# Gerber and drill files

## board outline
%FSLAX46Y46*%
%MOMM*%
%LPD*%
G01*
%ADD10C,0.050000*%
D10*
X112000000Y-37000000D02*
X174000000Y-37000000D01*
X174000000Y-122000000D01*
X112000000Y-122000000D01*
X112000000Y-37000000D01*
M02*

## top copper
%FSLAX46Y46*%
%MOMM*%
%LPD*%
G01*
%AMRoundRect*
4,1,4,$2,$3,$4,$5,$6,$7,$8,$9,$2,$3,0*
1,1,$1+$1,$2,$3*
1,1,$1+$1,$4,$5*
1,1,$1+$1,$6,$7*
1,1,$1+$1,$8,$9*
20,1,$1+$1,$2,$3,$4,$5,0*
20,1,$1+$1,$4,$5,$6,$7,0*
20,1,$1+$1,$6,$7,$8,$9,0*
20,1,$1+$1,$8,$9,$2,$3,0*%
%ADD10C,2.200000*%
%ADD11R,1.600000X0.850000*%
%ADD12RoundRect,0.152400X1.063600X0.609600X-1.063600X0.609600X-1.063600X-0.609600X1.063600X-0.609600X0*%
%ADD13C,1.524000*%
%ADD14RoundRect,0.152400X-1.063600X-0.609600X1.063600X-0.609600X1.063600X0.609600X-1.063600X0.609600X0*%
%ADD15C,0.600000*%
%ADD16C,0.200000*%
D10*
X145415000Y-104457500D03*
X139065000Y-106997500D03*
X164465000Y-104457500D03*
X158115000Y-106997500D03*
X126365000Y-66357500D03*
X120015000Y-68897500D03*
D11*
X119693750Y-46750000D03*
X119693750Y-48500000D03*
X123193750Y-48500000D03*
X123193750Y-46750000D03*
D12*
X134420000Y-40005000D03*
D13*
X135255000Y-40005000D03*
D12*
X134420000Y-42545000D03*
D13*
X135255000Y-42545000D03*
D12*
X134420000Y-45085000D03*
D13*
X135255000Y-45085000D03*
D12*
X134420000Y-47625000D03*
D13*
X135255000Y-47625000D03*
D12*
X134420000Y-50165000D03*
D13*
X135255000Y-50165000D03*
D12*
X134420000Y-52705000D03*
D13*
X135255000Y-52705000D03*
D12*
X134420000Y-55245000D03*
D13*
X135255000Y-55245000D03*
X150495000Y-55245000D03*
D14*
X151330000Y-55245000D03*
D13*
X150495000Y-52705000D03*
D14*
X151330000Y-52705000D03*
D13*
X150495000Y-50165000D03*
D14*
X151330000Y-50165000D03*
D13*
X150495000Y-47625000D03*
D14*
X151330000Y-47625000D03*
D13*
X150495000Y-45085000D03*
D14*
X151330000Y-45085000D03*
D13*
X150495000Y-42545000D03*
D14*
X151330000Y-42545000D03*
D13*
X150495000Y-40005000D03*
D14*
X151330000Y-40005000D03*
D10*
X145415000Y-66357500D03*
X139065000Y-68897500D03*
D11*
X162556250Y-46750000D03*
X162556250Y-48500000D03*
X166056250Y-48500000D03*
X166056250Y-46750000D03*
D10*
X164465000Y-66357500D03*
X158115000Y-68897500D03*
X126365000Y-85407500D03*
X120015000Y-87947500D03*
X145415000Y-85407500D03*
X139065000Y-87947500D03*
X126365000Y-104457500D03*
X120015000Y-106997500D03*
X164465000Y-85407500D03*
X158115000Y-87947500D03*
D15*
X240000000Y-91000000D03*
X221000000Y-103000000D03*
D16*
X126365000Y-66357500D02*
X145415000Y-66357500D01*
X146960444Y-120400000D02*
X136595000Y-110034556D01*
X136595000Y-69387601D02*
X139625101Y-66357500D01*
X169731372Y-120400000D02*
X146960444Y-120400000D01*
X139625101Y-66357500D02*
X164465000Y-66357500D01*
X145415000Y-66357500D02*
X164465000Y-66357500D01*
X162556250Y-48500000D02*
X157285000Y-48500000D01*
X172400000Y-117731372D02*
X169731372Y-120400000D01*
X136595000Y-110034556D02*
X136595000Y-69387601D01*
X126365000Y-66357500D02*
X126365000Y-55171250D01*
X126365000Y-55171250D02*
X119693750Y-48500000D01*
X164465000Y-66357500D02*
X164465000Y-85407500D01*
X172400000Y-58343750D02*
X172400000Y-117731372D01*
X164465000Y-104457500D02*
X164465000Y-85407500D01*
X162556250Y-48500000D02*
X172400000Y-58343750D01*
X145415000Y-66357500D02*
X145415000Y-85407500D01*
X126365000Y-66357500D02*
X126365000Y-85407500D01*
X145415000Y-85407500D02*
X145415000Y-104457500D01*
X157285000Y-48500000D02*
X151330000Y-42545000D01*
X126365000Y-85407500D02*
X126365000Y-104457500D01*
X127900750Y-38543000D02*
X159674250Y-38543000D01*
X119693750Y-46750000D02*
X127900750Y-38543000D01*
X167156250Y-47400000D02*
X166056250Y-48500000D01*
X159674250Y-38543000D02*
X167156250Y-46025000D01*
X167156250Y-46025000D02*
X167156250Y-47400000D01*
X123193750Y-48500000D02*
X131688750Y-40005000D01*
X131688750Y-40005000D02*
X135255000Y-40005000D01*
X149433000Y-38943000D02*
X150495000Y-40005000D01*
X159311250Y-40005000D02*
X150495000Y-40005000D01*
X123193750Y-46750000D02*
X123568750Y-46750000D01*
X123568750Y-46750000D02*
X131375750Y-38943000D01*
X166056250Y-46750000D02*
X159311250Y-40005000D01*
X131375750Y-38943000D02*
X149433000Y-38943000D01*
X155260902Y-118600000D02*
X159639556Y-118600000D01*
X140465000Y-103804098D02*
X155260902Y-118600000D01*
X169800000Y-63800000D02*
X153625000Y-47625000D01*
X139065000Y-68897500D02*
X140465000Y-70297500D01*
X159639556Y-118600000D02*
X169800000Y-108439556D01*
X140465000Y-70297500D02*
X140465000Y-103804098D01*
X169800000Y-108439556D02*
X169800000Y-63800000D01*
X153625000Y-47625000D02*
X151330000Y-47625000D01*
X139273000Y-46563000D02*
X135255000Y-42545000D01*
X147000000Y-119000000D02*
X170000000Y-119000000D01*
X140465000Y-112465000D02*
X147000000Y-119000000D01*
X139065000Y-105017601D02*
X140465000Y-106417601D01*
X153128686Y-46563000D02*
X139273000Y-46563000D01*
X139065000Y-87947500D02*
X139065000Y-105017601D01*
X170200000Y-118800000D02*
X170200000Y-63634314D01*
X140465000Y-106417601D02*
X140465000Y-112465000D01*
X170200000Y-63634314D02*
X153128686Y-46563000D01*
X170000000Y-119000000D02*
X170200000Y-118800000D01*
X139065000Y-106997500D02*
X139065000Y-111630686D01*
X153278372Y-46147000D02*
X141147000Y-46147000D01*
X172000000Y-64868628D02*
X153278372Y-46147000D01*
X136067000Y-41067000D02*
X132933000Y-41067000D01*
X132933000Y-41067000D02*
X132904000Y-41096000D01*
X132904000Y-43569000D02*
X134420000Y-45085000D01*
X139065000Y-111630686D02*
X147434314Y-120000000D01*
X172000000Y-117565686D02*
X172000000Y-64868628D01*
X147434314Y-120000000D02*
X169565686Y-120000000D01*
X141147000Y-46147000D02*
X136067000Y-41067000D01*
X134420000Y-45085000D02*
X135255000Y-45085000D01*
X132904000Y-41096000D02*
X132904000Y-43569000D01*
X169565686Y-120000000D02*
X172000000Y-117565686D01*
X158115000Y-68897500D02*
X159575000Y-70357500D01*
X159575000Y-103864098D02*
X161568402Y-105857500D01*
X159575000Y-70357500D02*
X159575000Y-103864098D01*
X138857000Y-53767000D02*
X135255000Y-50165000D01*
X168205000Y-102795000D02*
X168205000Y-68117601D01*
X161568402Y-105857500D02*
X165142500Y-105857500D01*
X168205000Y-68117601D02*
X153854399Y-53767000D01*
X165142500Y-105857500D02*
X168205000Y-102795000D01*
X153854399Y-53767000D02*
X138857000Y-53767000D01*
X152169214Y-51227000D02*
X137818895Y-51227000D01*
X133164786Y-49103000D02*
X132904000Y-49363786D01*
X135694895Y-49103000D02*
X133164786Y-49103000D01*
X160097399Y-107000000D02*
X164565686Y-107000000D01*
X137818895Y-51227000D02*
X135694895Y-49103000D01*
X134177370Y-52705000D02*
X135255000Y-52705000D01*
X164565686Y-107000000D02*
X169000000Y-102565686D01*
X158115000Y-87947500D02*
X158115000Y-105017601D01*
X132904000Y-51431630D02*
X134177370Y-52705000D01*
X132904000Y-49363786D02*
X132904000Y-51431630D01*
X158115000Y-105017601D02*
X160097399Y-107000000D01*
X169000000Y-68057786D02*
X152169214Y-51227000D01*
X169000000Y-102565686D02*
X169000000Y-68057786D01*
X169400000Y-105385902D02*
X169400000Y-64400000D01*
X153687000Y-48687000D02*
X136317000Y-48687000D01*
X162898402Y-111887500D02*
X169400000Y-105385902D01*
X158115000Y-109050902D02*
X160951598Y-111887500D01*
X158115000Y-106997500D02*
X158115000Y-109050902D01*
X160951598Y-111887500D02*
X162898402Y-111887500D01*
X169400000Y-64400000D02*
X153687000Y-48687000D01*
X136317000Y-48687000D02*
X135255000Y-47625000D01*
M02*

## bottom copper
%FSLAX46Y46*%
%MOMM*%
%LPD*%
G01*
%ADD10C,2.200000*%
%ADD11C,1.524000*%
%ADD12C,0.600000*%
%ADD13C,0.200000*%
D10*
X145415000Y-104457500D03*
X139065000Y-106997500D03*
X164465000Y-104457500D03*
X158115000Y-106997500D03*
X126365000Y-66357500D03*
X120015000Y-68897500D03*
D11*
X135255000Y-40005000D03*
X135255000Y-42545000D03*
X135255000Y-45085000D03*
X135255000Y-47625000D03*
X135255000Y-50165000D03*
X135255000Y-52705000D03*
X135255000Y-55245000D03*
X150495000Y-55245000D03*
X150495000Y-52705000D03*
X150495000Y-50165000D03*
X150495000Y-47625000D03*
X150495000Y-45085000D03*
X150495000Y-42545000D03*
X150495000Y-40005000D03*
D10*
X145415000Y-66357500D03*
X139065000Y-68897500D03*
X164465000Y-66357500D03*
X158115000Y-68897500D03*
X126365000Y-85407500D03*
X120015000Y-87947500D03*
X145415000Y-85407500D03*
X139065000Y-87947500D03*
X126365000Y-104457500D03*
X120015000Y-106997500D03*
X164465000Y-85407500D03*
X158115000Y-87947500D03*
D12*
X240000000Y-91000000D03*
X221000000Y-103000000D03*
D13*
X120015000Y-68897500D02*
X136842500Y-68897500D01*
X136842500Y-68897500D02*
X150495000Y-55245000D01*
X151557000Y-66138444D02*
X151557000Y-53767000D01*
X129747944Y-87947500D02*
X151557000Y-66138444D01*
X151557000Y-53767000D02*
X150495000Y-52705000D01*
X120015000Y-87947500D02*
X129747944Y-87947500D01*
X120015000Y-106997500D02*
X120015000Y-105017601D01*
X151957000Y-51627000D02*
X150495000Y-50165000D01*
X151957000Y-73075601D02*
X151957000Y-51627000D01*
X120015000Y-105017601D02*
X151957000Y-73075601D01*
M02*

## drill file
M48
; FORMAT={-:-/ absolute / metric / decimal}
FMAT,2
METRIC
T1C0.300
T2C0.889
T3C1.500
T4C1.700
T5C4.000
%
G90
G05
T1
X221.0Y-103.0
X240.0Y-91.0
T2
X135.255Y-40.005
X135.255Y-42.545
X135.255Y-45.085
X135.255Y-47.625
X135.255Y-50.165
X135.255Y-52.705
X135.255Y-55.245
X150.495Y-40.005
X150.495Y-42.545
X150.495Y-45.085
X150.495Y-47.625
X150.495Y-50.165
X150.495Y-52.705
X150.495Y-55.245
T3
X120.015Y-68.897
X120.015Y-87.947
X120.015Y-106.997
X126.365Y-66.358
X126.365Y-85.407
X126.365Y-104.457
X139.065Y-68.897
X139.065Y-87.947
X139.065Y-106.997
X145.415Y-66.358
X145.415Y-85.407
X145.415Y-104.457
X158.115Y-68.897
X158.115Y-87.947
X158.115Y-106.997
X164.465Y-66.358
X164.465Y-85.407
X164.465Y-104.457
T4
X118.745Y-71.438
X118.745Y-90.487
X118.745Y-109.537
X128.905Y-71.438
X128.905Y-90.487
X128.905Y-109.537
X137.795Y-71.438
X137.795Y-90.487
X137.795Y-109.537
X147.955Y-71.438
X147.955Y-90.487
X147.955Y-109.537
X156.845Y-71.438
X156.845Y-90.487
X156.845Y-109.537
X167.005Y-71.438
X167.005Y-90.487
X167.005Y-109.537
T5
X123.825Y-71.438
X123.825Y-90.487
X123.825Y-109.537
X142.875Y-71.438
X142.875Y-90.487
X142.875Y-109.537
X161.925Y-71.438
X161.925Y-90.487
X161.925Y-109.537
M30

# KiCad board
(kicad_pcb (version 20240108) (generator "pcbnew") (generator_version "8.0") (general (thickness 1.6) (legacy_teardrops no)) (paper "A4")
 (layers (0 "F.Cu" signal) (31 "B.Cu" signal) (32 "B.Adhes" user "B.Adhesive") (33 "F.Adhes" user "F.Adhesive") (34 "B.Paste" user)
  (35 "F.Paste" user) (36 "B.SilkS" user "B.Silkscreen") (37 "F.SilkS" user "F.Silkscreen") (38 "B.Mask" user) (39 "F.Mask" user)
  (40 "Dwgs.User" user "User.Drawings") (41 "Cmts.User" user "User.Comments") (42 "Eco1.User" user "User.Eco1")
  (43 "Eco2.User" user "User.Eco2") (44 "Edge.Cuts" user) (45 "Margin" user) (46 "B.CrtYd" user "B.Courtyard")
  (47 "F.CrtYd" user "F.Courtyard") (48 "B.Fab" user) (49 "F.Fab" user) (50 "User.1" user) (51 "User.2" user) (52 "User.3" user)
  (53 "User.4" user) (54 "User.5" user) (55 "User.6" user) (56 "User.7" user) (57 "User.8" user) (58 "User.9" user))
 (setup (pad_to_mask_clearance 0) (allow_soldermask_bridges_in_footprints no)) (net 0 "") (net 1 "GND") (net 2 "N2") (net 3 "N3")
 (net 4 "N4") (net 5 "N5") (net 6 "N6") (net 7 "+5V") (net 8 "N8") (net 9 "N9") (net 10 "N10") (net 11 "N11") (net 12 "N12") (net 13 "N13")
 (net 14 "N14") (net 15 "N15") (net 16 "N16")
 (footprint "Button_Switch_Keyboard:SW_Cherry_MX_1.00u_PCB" (layer "F.Cu") (at 145.415 104.4575)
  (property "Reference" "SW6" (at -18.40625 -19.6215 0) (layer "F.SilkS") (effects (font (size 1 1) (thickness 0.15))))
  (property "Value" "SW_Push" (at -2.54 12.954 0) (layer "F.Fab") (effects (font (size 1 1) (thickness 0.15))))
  (pad "" np_thru_hole circle (at -7.62 5.08) (size 1.7 1.7) (drill 1.7) (layers "*.Cu" "*.Mask"))
  (pad "" np_thru_hole circle (at -2.54 5.08) (size 4 4) (drill 4) (layers "*.Cu" "*.Mask"))
  (pad "" np_thru_hole circle (at 2.54 5.08) (size 1.7 1.7) (drill 1.7) (layers "*.Cu" "*.Mask"))
  (pad "1" thru_hole circle (at 0 0) (size 2.2 2.2) (drill 1.5) (layers "*.Cu" "*.Mask") (remove_unused_layers no) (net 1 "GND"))
  (pad "2" thru_hole circle (at -6.35 2.54) (size 2.2 2.2) (drill 1.5) (layers "*.Cu" "*.Mask") (remove_unused_layers no) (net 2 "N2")))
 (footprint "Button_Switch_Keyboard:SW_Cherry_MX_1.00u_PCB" (layer "F.Cu") (at 164.465 104.4575)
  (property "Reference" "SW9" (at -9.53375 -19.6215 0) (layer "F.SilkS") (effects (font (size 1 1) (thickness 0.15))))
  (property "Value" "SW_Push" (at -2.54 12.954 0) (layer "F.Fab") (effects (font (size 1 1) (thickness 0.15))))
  (pad "" np_thru_hole circle (at -7.62 5.08) (size 1.7 1.7) (drill 1.7) (layers "*.Cu" "*.Mask"))
  (pad "" np_thru_hole circle (at -2.54 5.08) (size 4 4) (drill 4) (layers "*.Cu" "*.Mask"))
  (pad "" np_thru_hole circle (at 2.54 5.08) (size 1.7 1.7) (drill 1.7) (layers "*.Cu" "*.Mask"))
  (pad "1" thru_hole circle (at 0 0) (size 2.2 2.2) (drill 1.5) (layers "*.Cu" "*.Mask") (remove_unused_layers no) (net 1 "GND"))
  (pad "2" thru_hole circle (at -6.35 2.54) (size 2.2 2.2) (drill 1.5) (layers "*.Cu" "*.Mask") (remove_unused_layers no) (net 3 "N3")))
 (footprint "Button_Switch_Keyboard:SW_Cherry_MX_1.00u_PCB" (layer "F.Cu") (at 126.365 66.3575)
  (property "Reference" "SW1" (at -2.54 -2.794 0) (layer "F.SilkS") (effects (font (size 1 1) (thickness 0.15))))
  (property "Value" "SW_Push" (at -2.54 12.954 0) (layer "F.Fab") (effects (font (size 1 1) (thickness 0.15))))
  (pad "" np_thru_hole circle (at -7.62 5.08) (size 1.7 1.7) (drill 1.7) (layers "*.Cu" "*.Mask"))
  (pad "" np_thru_hole circle (at -2.54 5.08) (size 4 4) (drill 4) (layers "*.Cu" "*.Mask"))
  (pad "" np_thru_hole circle (at 2.54 5.08) (size 1.7 1.7) (drill 1.7) (layers "*.Cu" "*.Mask"))
  (pad "1" thru_hole circle (at 0 0) (size 2.2 2.2) (drill 1.5) (layers "*.Cu" "*.Mask") (remove_unused_layers no) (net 1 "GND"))
  (pad "2" thru_hole circle (at -6.35 2.54) (size 2.2 2.2) (drill 1.5) (layers "*.Cu" "*.Mask") (remove_unused_layers no) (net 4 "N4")))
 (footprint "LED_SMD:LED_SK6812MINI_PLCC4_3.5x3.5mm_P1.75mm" (layer "F.Cu") (at 121.44375 47.625)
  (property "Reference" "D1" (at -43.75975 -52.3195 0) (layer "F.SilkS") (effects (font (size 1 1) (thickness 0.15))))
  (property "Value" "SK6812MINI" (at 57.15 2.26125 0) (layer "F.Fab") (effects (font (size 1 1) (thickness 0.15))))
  (pad "1" smd rect (at -1.75 -0.875) (size 1.6 0.85) (layers "F.Cu" "F.Paste" "F.Mask") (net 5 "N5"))
  (pad "2" smd rect (at -1.75 0.875) (size 1.6 0.85) (layers "F.Cu" "F.Paste" "F.Mask") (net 1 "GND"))
  (pad "3" smd rect (at 1.75 0.875) (size 1.6 0.85) (layers "F.Cu" "F.Paste" "F.Mask") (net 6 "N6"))
  (pad "4" smd rect (at 1.75 -0.875) (size 1.6 0.85) (layers "F.Cu" "F.Paste" "F.Mask") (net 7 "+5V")))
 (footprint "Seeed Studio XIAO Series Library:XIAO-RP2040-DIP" (layer "F.Cu") (at 142.875 47.625)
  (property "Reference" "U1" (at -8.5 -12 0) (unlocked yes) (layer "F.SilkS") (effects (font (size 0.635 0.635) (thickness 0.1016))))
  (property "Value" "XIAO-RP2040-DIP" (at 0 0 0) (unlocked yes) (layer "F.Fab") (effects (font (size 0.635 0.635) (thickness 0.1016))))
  (pad "1" smd roundrect (at -8.455 -7.62 180) (size 2.432 1.524) (layers "F.Cu" "F.Mask") (roundrect_rratio 0.1) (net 6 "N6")
   (thermal_bridge_angle 45))
  (pad "1" thru_hole circle (at -7.62 -7.62 180) (size 1.524 1.524) (drill 0.889) (layers "*.Cu" "*.Mask") (remove_unused_layers no)
   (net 6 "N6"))
  (pad "2" smd roundrect (at -8.455 -5.08 180) (size 2.432 1.524) (layers "F.Cu" "F.Mask") (roundrect_rratio 0.1) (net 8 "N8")
   (thermal_bridge_angle 45))
  (pad "2" thru_hole circle (at -7.62 -5.08 180) (size 1.524 1.524) (drill 0.889) (layers "*.Cu" "*.Mask") (remove_unused_layers no)
   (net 8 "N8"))
  (pad "3" smd roundrect (at -8.455 -2.54 180) (size 2.432 1.524) (layers "F.Cu" "F.Mask") (roundrect_rratio 0.1) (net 2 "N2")
   (thermal_bridge_angle 45))
  (pad "3" thru_hole circle (at -7.62 -2.54 180) (size 1.524 1.524) (drill 0.889) (layers "*.Cu" "*.Mask") (remove_unused_layers no)
   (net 2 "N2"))
  (pad "4" smd roundrect (at -8.455 0 180) (size 2.432 1.524) (layers "F.Cu" "F.Mask") (roundrect_rratio 0.1) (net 3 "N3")
   (thermal_bridge_angle 45))
  (pad "4" thru_hole circle (at -7.62 0 180) (size 1.524 1.524) (drill 0.889) (layers "*.Cu" "*.Mask") (remove_unused_layers no)
   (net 3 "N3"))
  (pad "5" smd roundrect (at -8.455 2.54 180) (size 2.432 1.524) (layers "F.Cu" "F.Mask") (roundrect_rratio 0.1) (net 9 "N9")
   (thermal_bridge_angle 45))
  (pad "5" thru_hole circle (at -7.62 2.54 180) (size 1.524 1.524) (drill 0.889) (layers "*.Cu" "*.Mask") (remove_unused_layers no)
   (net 9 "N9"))
  (pad "6" smd roundrect (at -8.455 5.08 180) (size 2.432 1.524) (layers "F.Cu" "F.Mask") (roundrect_rratio 0.1) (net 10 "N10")
   (thermal_bridge_angle 45))
  (pad "6" thru_hole circle (at -7.62 5.08 180) (size 1.524 1.524) (drill 0.889) (layers "*.Cu" "*.Mask") (remove_unused_layers no)
   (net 10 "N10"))
  (pad "7" smd roundrect (at -8.455 7.62 180) (size 2.432 1.524) (layers "F.Cu" "F.Mask") (roundrect_rratio 0.1) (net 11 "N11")
   (thermal_bridge_angle 45))
  (pad "7" thru_hole circle (at -7.62 7.62 180) (size 1.524 1.524) (drill 0.889) (layers "*.Cu" "*.Mask") (remove_unused_layers no)
   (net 11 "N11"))
  (pad "8" thru_hole circle (at 7.62 7.62) (size 1.524 1.524) (drill 0.889) (layers "*.Cu" "*.Mask") (remove_unused_layers no) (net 4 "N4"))
  (pad "8" smd roundrect (at 8.455 7.62) (size 2.432 1.524) (layers "F.Cu" "F.Mask") (roundrect_rratio 0.1) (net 4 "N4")
   (thermal_bridge_angle 45))
  (pad "9" thru_hole circle (at 7.62 5.08) (size 1.524 1.524) (drill 0.889) (layers "*.Cu" "*.Mask") (remove_unused_layers no)
   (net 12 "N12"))
  (pad "9" smd roundrect (at 8.455 5.08) (size 2.432 1.524) (layers "F.Cu" "F.Mask") (roundrect_rratio 0.1) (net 12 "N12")
   (thermal_bridge_angle 45))
  (pad "10" thru_hole circle (at 7.62 2.54) (size 1.524 1.524) (drill 0.889) (layers "*.Cu" "*.Mask") (remove_unused_layers no)
   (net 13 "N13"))
  (pad "10" smd roundrect (at 8.455 2.54) (size 2.432 1.524) (layers "F.Cu" "F.Mask") (roundrect_rratio 0.1) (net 13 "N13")
   (thermal_bridge_angle 45))
  (pad "11" thru_hole circle (at 7.62 0) (size 1.524 1.524) (drill 0.889) (layers "*.Cu" "*.Mask") (remove_unused_layers no) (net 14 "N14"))
  (pad "11" smd roundrect (at 8.455 0) (size 2.432 1.524) (layers "F.Cu" "F.Mask") (roundrect_rratio 0.1) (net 14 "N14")
   (thermal_bridge_angle 45))
  (pad "12" thru_hole circle (at 7.62 -2.54) (size 1.524 1.524) (drill 0.889) (layers "*.Cu" "*.Mask") (remove_unused_layers no)
   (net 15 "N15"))
  (pad "12" smd roundrect (at 8.455 -2.54) (size 2.432 1.524) (layers "F.Cu" "F.Mask") (roundrect_rratio 0.1) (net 15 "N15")
   (thermal_bridge_angle 45))
  (pad "13" thru_hole circle (at 7.62 -5.08) (size 1.524 1.524) (drill 0.889) (layers "*.Cu" "*.Mask") (remove_unused_layers no)
   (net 1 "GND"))
  (pad "13" smd roundrect (at 8.455 -5.08) (size 2.432 1.524) (layers "F.Cu" "F.Mask") (roundrect_rratio 0.1) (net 1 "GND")
   (thermal_bridge_angle 45))
  (pad "14" thru_hole circle (at 7.62 -7.62) (size 1.524 1.524) (drill 0.889) (layers "*.Cu" "*.Mask") (remove_unused_layers no)
   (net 7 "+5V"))
  (pad "14" smd roundrect (at 8.455 -7.62) (size 2.432 1.524) (layers "F.Cu" "F.Mask") (roundrect_rratio 0.1) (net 7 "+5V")
   (thermal_bridge_angle 45)))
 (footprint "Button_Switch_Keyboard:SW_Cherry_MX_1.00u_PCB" (layer "F.Cu") (at 145.415 66.3575)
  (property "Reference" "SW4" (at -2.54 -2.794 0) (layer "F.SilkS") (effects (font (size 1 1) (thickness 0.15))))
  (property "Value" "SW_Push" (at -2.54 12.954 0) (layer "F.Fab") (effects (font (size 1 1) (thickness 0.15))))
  (pad "" np_thru_hole circle (at -7.62 5.08) (size 1.7 1.7) (drill 1.7) (layers "*.Cu" "*.Mask"))
  (pad "" np_thru_hole circle (at -2.54 5.08) (size 4 4) (drill 4) (layers "*.Cu" "*.Mask"))
  (pad "" np_thru_hole circle (at 2.54 5.08) (size 1.7 1.7) (drill 1.7) (layers "*.Cu" "*.Mask"))
  (pad "1" thru_hole circle (at 0 0) (size 2.2 2.2) (drill 1.5) (layers "*.Cu" "*.Mask") (remove_unused_layers no) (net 1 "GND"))
  (pad "2" thru_hole circle (at -6.35 2.54) (size 2.2 2.2) (drill 1.5) (layers "*.Cu" "*.Mask") (remove_unused_layers no) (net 14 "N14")))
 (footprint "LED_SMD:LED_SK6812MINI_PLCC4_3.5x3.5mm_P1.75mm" (layer "F.Cu") (at 164.30625 47.625)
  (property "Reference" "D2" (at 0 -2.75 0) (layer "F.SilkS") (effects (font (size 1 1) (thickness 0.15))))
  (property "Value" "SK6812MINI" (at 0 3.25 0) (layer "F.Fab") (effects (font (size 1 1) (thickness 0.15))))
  (pad "1" smd rect (at -1.75 -0.875) (size 1.6 0.85) (layers "F.Cu" "F.Paste" "F.Mask") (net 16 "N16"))
  (pad "2" smd rect (at -1.75 0.875) (size 1.6 0.85) (layers "F.Cu" "F.Paste" "F.Mask") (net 1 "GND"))
  (pad "3" smd rect (at 1.75 0.875) (size 1.6 0.85) (layers "F.Cu" "F.Paste" "F.Mask") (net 5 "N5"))
  (pad "4" smd rect (at 1.75 -0.875) (size 1.6 0.85) (layers "F.Cu" "F.Paste" "F.Mask") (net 7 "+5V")))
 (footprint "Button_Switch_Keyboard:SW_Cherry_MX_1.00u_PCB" (layer "F.Cu") (at 164.465 66.3575)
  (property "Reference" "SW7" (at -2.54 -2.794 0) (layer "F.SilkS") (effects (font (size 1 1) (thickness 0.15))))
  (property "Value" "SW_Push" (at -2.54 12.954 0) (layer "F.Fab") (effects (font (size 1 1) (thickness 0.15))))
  (pad "" np_thru_hole circle (at -7.62 5.08) (size 1.7 1.7) (drill 1.7) (layers "*.Cu" "*.Mask"))
  (pad "" np_thru_hole circle (at -2.54 5.08) (size 4 4) (drill 4) (layers "*.Cu" "*.Mask"))
  (pad "" np_thru_hole circle (at 2.54 5.08) (size 1.7 1.7) (drill 1.7) (layers "*.Cu" "*.Mask"))
  (pad "1" thru_hole circle (at 0 0) (size 2.2 2.2) (drill 1.5) (layers "*.Cu" "*.Mask") (remove_unused_layers no) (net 1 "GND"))
  (pad "2" thru_hole circle (at -6.35 2.54) (size 2.2 2.2) (drill 1.5) (layers "*.Cu" "*.Mask") (remove_unused_layers no) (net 9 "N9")))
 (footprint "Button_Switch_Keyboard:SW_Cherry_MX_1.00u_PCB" (layer "F.Cu") (at 126.365 85.4075)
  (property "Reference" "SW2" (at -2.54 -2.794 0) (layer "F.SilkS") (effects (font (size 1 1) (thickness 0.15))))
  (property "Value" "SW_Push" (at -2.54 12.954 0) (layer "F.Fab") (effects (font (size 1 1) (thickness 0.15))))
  (pad "" np_thru_hole circle (at -7.62 5.08) (size 1.7 1.7) (drill 1.7) (layers "*.Cu" "*.Mask"))
  (pad "" np_thru_hole circle (at -2.54 5.08) (size 4 4) (drill 4) (layers "*.Cu" "*.Mask"))
  (pad "" np_thru_hole circle (at 2.54 5.08) (size 1.7 1.7) (drill 1.7) (layers "*.Cu" "*.Mask"))
  (pad "1" thru_hole circle (at 0 0) (size 2.2 2.2) (drill 1.5) (layers "*.Cu" "*.Mask") (remove_unused_layers no) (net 1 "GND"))
  (pad "2" thru_hole circle (at -6.35 2.54) (size 2.2 2.2) (drill 1.5) (layers "*.Cu" "*.Mask") (remove_unused_layers no) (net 12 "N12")))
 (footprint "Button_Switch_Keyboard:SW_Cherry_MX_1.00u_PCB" (layer "F.Cu") (at 145.415 85.4075)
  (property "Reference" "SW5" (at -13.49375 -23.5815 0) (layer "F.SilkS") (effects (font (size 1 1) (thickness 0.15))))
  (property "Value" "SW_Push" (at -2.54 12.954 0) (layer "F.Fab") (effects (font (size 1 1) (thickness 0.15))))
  (pad "" np_thru_hole circle (at -7.62 5.08) (size 1.7 1.7) (drill 1.7) (layers "*.Cu" "*.Mask"))
  (pad "" np_thru_hole circle (at -2.54 5.08) (size 4 4) (drill 4) (layers "*.Cu" "*.Mask"))
  (pad "" np_thru_hole circle (at 2.54 5.08) (size 1.7 1.7) (drill 1.7) (layers "*.Cu" "*.Mask"))
  (pad "1" thru_hole circle (at 0 0) (size 2.2 2.2) (drill 1.5) (layers "*.Cu" "*.Mask") (remove_unused_layers no) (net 1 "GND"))
  (pad "2" thru_hole circle (at -6.35 2.54) (size 2.2 2.2) (drill 1.5) (layers "*.Cu" "*.Mask") (remove_unused_layers no) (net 8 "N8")))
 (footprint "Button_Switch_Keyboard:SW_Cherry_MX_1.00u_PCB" (layer "F.Cu") (at 126.365 104.4575)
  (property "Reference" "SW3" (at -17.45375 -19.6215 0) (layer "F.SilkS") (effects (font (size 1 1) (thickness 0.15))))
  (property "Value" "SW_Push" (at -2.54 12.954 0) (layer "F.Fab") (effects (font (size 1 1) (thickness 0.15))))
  (pad "" np_thru_hole circle (at -7.62 5.08) (size 1.7 1.7) (drill 1.7) (layers "*.Cu" "*.Mask"))
  (pad "" np_thru_hole circle (at -2.54 5.08) (size 4 4) (drill 4) (layers "*.Cu" "*.Mask"))
  (pad "" np_thru_hole circle (at 2.54 5.08) (size 1.7 1.7) (drill 1.7) (layers "*.Cu" "*.Mask"))
  (pad "1" thru_hole circle (at 0 0) (size 2.2 2.2) (drill 1.5) (layers "*.Cu" "*.Mask") (remove_unused_layers no) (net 1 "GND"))
  (pad "2" thru_hole circle (at -6.35 2.54) (size 2.2 2.2) (drill 1.5) (layers "*.Cu" "*.Mask") (remove_unused_layers no) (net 13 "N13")))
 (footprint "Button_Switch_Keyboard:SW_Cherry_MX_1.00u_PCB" (layer "F.Cu") (at 164.465 85.4075)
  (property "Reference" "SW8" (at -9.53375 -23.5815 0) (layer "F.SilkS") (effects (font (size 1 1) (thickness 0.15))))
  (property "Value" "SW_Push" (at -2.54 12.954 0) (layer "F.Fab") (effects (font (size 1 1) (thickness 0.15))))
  (pad "" np_thru_hole circle (at -7.62 5.08) (size 1.7 1.7) (drill 1.7) (layers "*.Cu" "*.Mask"))
  (pad "" np_thru_hole circle (at -2.54 5.08) (size 4 4) (drill 4) (layers "*.Cu" "*.Mask"))
  (pad "" np_thru_hole circle (at 2.54 5.08) (size 1.7 1.7) (drill 1.7) (layers "*.Cu" "*.Mask"))
  (pad "1" thru_hole circle (at 0 0) (size 2.2 2.2) (drill 1.5) (layers "*.Cu" "*.Mask") (remove_unused_layers no) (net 1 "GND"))
  (pad "2" thru_hole circle (at -6.35 2.54) (size 2.2 2.2) (drill 1.5) (layers "*.Cu" "*.Mask") (remove_unused_layers no) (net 10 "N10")))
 (gr_rect (start 112 37) (end 174 122) (stroke (width 0.05) (type default)) (fill none) (layer "Edge.Cuts"))
 (via (at 240 91) (size 0.6) (drill 0.3) (layers "F.Cu" "B.Cu") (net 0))
 (via (at 221 103) (size 0.6) (drill 0.3) (layers "F.Cu" "B.Cu") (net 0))
 (segment (start 126.365 66.3575) (end 145.415 66.3575) (width 0.2) (layer "F.Cu") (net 1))
 (segment (start 146.960444 120.4) (end 136.595 110.034556) (width 0.2) (layer "F.Cu") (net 1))
 (segment (start 136.595 69.387601) (end 139.625101 66.3575) (width 0.2) (layer "F.Cu") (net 1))
 (segment (start 169.731372 120.4) (end 146.960444 120.4) (width 0.2) (layer "F.Cu") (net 1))
 (segment (start 139.625101 66.3575) (end 164.465 66.3575) (width 0.2) (layer "F.Cu") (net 1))
 (segment (start 145.415 66.3575) (end 164.465 66.3575) (width 0.2) (layer "F.Cu") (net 1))
 (segment (start 162.55625 48.5) (end 157.285 48.5) (width 0.2) (layer "F.Cu") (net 1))
 (segment (start 172.4 117.731372) (end 169.731372 120.4) (width 0.2) (layer "F.Cu") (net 1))
 (segment (start 136.595 110.034556) (end 136.595 69.387601) (width 0.2) (layer "F.Cu") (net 1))
 (segment (start 126.365 66.3575) (end 126.365 55.17125) (width 0.2) (layer "F.Cu") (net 1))
 (segment (start 126.365 55.17125) (end 119.69375 48.5) (width 0.2) (layer "F.Cu") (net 1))
 (segment (start 164.465 66.3575) (end 164.465 85.4075) (width 0.2) (layer "F.Cu") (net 1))
 (segment (start 172.4 58.34375) (end 172.4 117.731372) (width 0.2) (layer "F.Cu") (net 1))
 (segment (start 164.465 104.4575) (end 164.465 85.4075) (width 0.2) (layer "F.Cu") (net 1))
 (segment (start 162.55625 48.5) (end 172.4 58.34375) (width 0.2) (layer "F.Cu") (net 1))
 (segment (start 145.415 66.3575) (end 145.415 85.4075) (width 0.2) (layer "F.Cu") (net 1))
 (segment (start 126.365 66.3575) (end 126.365 85.4075) (width 0.2) (layer "F.Cu") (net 1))
 (segment (start 145.415 85.4075) (end 145.415 104.4575) (width 0.2) (layer "F.Cu") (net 1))
 (segment (start 157.285 48.5) (end 151.33 42.545) (width 0.2) (layer "F.Cu") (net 1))
 (segment (start 126.365 85.4075) (end 126.365 104.4575) (width 0.2) (layer "F.Cu") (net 1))
 (segment (start 127.90075 38.543) (end 159.67425 38.543) (width 0.2) (layer "F.Cu") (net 5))
 (segment (start 119.69375 46.75) (end 127.90075 38.543) (width 0.2) (layer "F.Cu") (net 5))
 (segment (start 167.15625 47.4) (end 166.05625 48.5) (width 0.2) (layer "F.Cu") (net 5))
 (segment (start 159.67425 38.543) (end 167.15625 46.025) (width 0.2) (layer "F.Cu") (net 5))
 (segment (start 167.15625 46.025) (end 167.15625 47.4) (width 0.2) (layer "F.Cu") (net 5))
 (segment (start 123.19375 48.5) (end 131.68875 40.005) (width 0.2) (layer "F.Cu") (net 6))
 (segment (start 131.68875 40.005) (end 135.255 40.005) (width 0.2) (layer "F.Cu") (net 6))
 (segment (start 149.433 38.943) (end 150.495 40.005) (width 0.2) (layer "F.Cu") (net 7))
 (segment (start 159.31125 40.005) (end 150.495 40.005) (width 0.2) (layer "F.Cu") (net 7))
 (segment (start 123.19375 46.75) (end 123.56875 46.75) (width 0.2) (layer "F.Cu") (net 7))
 (segment (start 123.56875 46.75) (end 131.37575 38.943) (width 0.2) (layer "F.Cu") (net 7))
 (segment (start 166.05625 46.75) (end 159.31125 40.005) (width 0.2) (layer "F.Cu") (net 7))
 (segment (start 131.37575 38.943) (end 149.433 38.943) (width 0.2) (layer "F.Cu") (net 7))
 (segment (start 120.015 68.8975) (end 136.8425 68.8975) (width 0.2) (layer "B.Cu") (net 4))
 (segment (start 136.8425 68.8975) (end 150.495 55.245) (width 0.2) (layer "B.Cu") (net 4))
 (segment (start 151.557 66.138444) (end 151.557 53.767) (width 0.2) (layer "B.Cu") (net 12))
 (segment (start 129.747944 87.9475) (end 151.557 66.138444) (width 0.2) (layer "B.Cu") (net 12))
 (segment (start 151.557 53.767) (end 150.495 52.705) (width 0.2) (layer "B.Cu") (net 12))
 (segment (start 120.015 87.9475) (end 129.747944 87.9475) (width 0.2) (layer "B.Cu") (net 12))
 (segment (start 120.015 106.9975) (end 120.015 105.017601) (width 0.2) (layer "B.Cu") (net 13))
 (segment (start 151.957 51.627) (end 150.495 50.165) (width 0.2) (layer "B.Cu") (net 13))
 (segment (start 151.957 73.075601) (end 151.957 51.627) (width 0.2) (layer "B.Cu") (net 13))
 (segment (start 120.015 105.017601) (end 151.957 73.075601) (width 0.2) (layer "B.Cu") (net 13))
 (segment (start 155.260902 118.6) (end 159.639556 118.6) (width 0.2) (layer "F.Cu") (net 14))
 (segment (start 140.465 103.804098) (end 155.260902 118.6) (width 0.2) (layer "F.Cu") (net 14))
 (segment (start 169.8 63.8) (end 153.625 47.625) (width 0.2) (layer "F.Cu") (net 14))
 (segment (start 139.065 68.8975) (end 140.465 70.2975) (width 0.2) (layer "F.Cu") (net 14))
 (segment (start 159.639556 118.6) (end 169.8 108.439556) (width 0.2) (layer "F.Cu") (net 14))
 (segment (start 140.465 70.2975) (end 140.465 103.804098) (width 0.2) (layer "F.Cu") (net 14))
 (segment (start 169.8 108.439556) (end 169.8 63.8) (width 0.2) (layer "F.Cu") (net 14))
 (segment (start 153.625 47.625) (end 151.33 47.625) (width 0.2) (layer "F.Cu") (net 14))
 (segment (start 139.273 46.563) (end 135.255 42.545) (width 0.2) (layer "F.Cu") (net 8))
 (segment (start 147 119) (end 170 119) (width 0.2) (layer "F.Cu") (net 8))
 (segment (start 140.465 112.465) (end 147 119) (width 0.2) (layer "F.Cu") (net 8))
 (segment (start 139.065 105.017601) (end 140.465 106.417601) (width 0.2) (layer "F.Cu") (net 8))
 (segment (start 153.128686 46.563) (end 139.273 46.563) (width 0.2) (layer "F.Cu") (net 8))
 (segment (start 139.065 87.9475) (end 139.065 105.017601) (width 0.2) (layer "F.Cu") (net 8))
 (segment (start 170.2 118.8) (end 170.2 63.634314) (width 0.2) (layer "F.Cu") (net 8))
 (segment (start 140.465 106.417601) (end 140.465 112.465) (width 0.2) (layer "F.Cu") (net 8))
 (segment (start 170.2 63.634314) (end 153.128686 46.563) (width 0.2) (layer "F.Cu") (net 8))
 (segment (start 170 119) (end 170.2 118.8) (width 0.2) (layer "F.Cu") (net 8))
 (segment (start 139.065 106.9975) (end 139.065 111.630686) (width 0.2) (layer "F.Cu") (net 2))
 (segment (start 153.278372 46.147) (end 141.147 46.147) (width 0.2) (layer "F.Cu") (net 2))
 (segment (start 172 64.868628) (end 153.278372 46.147) (width 0.2) (layer "F.Cu") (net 2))
 (segment (start 136.067 41.067) (end 132.933 41.067) (width 0.2) (layer "F.Cu") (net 2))
 (segment (start 132.933 41.067) (end 132.904 41.096) (width 0.2) (layer "F.Cu") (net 2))
 (segment (start 132.904 43.569) (end 134.42 45.085) (width 0.2) (layer "F.Cu") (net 2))
 (segment (start 139.065 111.630686) (end 147.434314 120) (width 0.2) (layer "F.Cu") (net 2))
 (segment (start 172 117.565686) (end 172 64.868628) (width 0.2) (layer "F.Cu") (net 2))
 (segment (start 147.434314 120) (end 169.565686 120) (width 0.2) (layer "F.Cu") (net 2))
 (segment (start 141.147 46.147) (end 136.067 41.067) (width 0.2) (layer "F.Cu") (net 2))
 (segment (start 134.42 45.085) (end 135.255 45.085) (width 0.2) (layer "F.Cu") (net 2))
 (segment (start 132.904 41.096) (end 132.904 43.569) (width 0.2) (layer "F.Cu") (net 2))
 (segment (start 169.565686 120) (end 172 117.565686) (width 0.2) (layer "F.Cu") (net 2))
 (segment (start 158.115 68.8975) (end 159.575 70.3575) (width 0.2) (layer "F.Cu") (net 9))
 (segment (start 159.575 103.864098) (end 161.568402 105.8575) (width 0.2) (layer "F.Cu") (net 9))
 (segment (start 159.575 70.3575) (end 159.575 103.864098) (width 0.2) (layer "F.Cu") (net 9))
 (segment (start 138.857 53.767) (end 135.255 50.165) (width 0.2) (layer "F.Cu") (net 9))
 (segment (start 168.205 102.795) (end 168.205 68.117601) (width 0.2) (layer "F.Cu") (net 9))
 (segment (start 161.568402 105.8575) (end 165.1425 105.8575) (width 0.2) (layer "F.Cu") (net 9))
 (segment (start 168.205 68.117601) (end 153.854399 53.767) (width 0.2) (layer "F.Cu") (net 9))
 (segment (start 165.1425 105.8575) (end 168.205 102.795) (width 0.2) (layer "F.Cu") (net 9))
 (segment (start 153.854399 53.767) (end 138.857 53.767) (width 0.2) (layer "F.Cu") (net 9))
 (segment (start 152.169214 51.227) (end 137.818895 51.227) (width 0.2) (layer "F.Cu") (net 10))
 (segment (start 133.164786 49.103) (end 132.904 49.363786) (width 0.2) (layer "F.Cu") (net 10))
 (segment (start 135.694895 49.103) (end 133.164786 49.103) (width 0.2) (layer "F.Cu") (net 10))
 (segment (start 160.097399 107) (end 164.565686 107) (width 0.2) (layer "F.Cu") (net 10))
 (segment (start 137.818895 51.227) (end 135.694895 49.103) (width 0.2) (layer "F.Cu") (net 10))
 (segment (start 134.17737 52.705) (end 135.255 52.705) (width 0.2) (layer "F.Cu") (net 10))
 (segment (start 164.565686 107) (end 169 102.565686) (width 0.2) (layer "F.Cu") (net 10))
 (segment (start 158.115 87.9475) (end 158.115 105.017601) (width 0.2) (layer "F.Cu") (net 10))
 (segment (start 132.904 51.43163) (end 134.17737 52.705) (width 0.2) (layer "F.Cu") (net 10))
 (segment (start 132.904 49.363786) (end 132.904 51.43163) (width 0.2) (layer "F.Cu") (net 10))
 (segment (start 158.115 105.017601) (end 160.097399 107) (width 0.2) (layer "F.Cu") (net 10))
 (segment (start 169 68.057786) (end 152.169214 51.227) (width 0.2) (layer "F.Cu") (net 10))
 (segment (start 169 102.565686) (end 169 68.057786) (width 0.2) (layer "F.Cu") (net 10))
 (segment (start 169.4 105.385902) (end 169.4 64.4) (width 0.2) (layer "F.Cu") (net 3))
 (segment (start 153.687 48.687) (end 136.317 48.687) (width 0.2) (layer "F.Cu") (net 3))
 (segment (start 162.898402 111.8875) (end 169.4 105.385902) (width 0.2) (layer "F.Cu") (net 3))
 (segment (start 158.115 109.050902) (end 160.951598 111.8875) (width 0.2) (layer "F.Cu") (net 3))
 (segment (start 158.115 106.9975) (end 158.115 109.050902) (width 0.2) (layer "F.Cu") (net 3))
 (segment (start 160.951598 111.8875) (end 162.898402 111.8875) (width 0.2) (layer "F.Cu") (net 3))
 (segment (start 169.4 64.4) (end 153.687 48.687) (width 0.2) (layer "F.Cu") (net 3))
 (segment (start 136.317 48.687) (end 135.255 47.625) (width 0.2) (layer "F.Cu") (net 3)))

